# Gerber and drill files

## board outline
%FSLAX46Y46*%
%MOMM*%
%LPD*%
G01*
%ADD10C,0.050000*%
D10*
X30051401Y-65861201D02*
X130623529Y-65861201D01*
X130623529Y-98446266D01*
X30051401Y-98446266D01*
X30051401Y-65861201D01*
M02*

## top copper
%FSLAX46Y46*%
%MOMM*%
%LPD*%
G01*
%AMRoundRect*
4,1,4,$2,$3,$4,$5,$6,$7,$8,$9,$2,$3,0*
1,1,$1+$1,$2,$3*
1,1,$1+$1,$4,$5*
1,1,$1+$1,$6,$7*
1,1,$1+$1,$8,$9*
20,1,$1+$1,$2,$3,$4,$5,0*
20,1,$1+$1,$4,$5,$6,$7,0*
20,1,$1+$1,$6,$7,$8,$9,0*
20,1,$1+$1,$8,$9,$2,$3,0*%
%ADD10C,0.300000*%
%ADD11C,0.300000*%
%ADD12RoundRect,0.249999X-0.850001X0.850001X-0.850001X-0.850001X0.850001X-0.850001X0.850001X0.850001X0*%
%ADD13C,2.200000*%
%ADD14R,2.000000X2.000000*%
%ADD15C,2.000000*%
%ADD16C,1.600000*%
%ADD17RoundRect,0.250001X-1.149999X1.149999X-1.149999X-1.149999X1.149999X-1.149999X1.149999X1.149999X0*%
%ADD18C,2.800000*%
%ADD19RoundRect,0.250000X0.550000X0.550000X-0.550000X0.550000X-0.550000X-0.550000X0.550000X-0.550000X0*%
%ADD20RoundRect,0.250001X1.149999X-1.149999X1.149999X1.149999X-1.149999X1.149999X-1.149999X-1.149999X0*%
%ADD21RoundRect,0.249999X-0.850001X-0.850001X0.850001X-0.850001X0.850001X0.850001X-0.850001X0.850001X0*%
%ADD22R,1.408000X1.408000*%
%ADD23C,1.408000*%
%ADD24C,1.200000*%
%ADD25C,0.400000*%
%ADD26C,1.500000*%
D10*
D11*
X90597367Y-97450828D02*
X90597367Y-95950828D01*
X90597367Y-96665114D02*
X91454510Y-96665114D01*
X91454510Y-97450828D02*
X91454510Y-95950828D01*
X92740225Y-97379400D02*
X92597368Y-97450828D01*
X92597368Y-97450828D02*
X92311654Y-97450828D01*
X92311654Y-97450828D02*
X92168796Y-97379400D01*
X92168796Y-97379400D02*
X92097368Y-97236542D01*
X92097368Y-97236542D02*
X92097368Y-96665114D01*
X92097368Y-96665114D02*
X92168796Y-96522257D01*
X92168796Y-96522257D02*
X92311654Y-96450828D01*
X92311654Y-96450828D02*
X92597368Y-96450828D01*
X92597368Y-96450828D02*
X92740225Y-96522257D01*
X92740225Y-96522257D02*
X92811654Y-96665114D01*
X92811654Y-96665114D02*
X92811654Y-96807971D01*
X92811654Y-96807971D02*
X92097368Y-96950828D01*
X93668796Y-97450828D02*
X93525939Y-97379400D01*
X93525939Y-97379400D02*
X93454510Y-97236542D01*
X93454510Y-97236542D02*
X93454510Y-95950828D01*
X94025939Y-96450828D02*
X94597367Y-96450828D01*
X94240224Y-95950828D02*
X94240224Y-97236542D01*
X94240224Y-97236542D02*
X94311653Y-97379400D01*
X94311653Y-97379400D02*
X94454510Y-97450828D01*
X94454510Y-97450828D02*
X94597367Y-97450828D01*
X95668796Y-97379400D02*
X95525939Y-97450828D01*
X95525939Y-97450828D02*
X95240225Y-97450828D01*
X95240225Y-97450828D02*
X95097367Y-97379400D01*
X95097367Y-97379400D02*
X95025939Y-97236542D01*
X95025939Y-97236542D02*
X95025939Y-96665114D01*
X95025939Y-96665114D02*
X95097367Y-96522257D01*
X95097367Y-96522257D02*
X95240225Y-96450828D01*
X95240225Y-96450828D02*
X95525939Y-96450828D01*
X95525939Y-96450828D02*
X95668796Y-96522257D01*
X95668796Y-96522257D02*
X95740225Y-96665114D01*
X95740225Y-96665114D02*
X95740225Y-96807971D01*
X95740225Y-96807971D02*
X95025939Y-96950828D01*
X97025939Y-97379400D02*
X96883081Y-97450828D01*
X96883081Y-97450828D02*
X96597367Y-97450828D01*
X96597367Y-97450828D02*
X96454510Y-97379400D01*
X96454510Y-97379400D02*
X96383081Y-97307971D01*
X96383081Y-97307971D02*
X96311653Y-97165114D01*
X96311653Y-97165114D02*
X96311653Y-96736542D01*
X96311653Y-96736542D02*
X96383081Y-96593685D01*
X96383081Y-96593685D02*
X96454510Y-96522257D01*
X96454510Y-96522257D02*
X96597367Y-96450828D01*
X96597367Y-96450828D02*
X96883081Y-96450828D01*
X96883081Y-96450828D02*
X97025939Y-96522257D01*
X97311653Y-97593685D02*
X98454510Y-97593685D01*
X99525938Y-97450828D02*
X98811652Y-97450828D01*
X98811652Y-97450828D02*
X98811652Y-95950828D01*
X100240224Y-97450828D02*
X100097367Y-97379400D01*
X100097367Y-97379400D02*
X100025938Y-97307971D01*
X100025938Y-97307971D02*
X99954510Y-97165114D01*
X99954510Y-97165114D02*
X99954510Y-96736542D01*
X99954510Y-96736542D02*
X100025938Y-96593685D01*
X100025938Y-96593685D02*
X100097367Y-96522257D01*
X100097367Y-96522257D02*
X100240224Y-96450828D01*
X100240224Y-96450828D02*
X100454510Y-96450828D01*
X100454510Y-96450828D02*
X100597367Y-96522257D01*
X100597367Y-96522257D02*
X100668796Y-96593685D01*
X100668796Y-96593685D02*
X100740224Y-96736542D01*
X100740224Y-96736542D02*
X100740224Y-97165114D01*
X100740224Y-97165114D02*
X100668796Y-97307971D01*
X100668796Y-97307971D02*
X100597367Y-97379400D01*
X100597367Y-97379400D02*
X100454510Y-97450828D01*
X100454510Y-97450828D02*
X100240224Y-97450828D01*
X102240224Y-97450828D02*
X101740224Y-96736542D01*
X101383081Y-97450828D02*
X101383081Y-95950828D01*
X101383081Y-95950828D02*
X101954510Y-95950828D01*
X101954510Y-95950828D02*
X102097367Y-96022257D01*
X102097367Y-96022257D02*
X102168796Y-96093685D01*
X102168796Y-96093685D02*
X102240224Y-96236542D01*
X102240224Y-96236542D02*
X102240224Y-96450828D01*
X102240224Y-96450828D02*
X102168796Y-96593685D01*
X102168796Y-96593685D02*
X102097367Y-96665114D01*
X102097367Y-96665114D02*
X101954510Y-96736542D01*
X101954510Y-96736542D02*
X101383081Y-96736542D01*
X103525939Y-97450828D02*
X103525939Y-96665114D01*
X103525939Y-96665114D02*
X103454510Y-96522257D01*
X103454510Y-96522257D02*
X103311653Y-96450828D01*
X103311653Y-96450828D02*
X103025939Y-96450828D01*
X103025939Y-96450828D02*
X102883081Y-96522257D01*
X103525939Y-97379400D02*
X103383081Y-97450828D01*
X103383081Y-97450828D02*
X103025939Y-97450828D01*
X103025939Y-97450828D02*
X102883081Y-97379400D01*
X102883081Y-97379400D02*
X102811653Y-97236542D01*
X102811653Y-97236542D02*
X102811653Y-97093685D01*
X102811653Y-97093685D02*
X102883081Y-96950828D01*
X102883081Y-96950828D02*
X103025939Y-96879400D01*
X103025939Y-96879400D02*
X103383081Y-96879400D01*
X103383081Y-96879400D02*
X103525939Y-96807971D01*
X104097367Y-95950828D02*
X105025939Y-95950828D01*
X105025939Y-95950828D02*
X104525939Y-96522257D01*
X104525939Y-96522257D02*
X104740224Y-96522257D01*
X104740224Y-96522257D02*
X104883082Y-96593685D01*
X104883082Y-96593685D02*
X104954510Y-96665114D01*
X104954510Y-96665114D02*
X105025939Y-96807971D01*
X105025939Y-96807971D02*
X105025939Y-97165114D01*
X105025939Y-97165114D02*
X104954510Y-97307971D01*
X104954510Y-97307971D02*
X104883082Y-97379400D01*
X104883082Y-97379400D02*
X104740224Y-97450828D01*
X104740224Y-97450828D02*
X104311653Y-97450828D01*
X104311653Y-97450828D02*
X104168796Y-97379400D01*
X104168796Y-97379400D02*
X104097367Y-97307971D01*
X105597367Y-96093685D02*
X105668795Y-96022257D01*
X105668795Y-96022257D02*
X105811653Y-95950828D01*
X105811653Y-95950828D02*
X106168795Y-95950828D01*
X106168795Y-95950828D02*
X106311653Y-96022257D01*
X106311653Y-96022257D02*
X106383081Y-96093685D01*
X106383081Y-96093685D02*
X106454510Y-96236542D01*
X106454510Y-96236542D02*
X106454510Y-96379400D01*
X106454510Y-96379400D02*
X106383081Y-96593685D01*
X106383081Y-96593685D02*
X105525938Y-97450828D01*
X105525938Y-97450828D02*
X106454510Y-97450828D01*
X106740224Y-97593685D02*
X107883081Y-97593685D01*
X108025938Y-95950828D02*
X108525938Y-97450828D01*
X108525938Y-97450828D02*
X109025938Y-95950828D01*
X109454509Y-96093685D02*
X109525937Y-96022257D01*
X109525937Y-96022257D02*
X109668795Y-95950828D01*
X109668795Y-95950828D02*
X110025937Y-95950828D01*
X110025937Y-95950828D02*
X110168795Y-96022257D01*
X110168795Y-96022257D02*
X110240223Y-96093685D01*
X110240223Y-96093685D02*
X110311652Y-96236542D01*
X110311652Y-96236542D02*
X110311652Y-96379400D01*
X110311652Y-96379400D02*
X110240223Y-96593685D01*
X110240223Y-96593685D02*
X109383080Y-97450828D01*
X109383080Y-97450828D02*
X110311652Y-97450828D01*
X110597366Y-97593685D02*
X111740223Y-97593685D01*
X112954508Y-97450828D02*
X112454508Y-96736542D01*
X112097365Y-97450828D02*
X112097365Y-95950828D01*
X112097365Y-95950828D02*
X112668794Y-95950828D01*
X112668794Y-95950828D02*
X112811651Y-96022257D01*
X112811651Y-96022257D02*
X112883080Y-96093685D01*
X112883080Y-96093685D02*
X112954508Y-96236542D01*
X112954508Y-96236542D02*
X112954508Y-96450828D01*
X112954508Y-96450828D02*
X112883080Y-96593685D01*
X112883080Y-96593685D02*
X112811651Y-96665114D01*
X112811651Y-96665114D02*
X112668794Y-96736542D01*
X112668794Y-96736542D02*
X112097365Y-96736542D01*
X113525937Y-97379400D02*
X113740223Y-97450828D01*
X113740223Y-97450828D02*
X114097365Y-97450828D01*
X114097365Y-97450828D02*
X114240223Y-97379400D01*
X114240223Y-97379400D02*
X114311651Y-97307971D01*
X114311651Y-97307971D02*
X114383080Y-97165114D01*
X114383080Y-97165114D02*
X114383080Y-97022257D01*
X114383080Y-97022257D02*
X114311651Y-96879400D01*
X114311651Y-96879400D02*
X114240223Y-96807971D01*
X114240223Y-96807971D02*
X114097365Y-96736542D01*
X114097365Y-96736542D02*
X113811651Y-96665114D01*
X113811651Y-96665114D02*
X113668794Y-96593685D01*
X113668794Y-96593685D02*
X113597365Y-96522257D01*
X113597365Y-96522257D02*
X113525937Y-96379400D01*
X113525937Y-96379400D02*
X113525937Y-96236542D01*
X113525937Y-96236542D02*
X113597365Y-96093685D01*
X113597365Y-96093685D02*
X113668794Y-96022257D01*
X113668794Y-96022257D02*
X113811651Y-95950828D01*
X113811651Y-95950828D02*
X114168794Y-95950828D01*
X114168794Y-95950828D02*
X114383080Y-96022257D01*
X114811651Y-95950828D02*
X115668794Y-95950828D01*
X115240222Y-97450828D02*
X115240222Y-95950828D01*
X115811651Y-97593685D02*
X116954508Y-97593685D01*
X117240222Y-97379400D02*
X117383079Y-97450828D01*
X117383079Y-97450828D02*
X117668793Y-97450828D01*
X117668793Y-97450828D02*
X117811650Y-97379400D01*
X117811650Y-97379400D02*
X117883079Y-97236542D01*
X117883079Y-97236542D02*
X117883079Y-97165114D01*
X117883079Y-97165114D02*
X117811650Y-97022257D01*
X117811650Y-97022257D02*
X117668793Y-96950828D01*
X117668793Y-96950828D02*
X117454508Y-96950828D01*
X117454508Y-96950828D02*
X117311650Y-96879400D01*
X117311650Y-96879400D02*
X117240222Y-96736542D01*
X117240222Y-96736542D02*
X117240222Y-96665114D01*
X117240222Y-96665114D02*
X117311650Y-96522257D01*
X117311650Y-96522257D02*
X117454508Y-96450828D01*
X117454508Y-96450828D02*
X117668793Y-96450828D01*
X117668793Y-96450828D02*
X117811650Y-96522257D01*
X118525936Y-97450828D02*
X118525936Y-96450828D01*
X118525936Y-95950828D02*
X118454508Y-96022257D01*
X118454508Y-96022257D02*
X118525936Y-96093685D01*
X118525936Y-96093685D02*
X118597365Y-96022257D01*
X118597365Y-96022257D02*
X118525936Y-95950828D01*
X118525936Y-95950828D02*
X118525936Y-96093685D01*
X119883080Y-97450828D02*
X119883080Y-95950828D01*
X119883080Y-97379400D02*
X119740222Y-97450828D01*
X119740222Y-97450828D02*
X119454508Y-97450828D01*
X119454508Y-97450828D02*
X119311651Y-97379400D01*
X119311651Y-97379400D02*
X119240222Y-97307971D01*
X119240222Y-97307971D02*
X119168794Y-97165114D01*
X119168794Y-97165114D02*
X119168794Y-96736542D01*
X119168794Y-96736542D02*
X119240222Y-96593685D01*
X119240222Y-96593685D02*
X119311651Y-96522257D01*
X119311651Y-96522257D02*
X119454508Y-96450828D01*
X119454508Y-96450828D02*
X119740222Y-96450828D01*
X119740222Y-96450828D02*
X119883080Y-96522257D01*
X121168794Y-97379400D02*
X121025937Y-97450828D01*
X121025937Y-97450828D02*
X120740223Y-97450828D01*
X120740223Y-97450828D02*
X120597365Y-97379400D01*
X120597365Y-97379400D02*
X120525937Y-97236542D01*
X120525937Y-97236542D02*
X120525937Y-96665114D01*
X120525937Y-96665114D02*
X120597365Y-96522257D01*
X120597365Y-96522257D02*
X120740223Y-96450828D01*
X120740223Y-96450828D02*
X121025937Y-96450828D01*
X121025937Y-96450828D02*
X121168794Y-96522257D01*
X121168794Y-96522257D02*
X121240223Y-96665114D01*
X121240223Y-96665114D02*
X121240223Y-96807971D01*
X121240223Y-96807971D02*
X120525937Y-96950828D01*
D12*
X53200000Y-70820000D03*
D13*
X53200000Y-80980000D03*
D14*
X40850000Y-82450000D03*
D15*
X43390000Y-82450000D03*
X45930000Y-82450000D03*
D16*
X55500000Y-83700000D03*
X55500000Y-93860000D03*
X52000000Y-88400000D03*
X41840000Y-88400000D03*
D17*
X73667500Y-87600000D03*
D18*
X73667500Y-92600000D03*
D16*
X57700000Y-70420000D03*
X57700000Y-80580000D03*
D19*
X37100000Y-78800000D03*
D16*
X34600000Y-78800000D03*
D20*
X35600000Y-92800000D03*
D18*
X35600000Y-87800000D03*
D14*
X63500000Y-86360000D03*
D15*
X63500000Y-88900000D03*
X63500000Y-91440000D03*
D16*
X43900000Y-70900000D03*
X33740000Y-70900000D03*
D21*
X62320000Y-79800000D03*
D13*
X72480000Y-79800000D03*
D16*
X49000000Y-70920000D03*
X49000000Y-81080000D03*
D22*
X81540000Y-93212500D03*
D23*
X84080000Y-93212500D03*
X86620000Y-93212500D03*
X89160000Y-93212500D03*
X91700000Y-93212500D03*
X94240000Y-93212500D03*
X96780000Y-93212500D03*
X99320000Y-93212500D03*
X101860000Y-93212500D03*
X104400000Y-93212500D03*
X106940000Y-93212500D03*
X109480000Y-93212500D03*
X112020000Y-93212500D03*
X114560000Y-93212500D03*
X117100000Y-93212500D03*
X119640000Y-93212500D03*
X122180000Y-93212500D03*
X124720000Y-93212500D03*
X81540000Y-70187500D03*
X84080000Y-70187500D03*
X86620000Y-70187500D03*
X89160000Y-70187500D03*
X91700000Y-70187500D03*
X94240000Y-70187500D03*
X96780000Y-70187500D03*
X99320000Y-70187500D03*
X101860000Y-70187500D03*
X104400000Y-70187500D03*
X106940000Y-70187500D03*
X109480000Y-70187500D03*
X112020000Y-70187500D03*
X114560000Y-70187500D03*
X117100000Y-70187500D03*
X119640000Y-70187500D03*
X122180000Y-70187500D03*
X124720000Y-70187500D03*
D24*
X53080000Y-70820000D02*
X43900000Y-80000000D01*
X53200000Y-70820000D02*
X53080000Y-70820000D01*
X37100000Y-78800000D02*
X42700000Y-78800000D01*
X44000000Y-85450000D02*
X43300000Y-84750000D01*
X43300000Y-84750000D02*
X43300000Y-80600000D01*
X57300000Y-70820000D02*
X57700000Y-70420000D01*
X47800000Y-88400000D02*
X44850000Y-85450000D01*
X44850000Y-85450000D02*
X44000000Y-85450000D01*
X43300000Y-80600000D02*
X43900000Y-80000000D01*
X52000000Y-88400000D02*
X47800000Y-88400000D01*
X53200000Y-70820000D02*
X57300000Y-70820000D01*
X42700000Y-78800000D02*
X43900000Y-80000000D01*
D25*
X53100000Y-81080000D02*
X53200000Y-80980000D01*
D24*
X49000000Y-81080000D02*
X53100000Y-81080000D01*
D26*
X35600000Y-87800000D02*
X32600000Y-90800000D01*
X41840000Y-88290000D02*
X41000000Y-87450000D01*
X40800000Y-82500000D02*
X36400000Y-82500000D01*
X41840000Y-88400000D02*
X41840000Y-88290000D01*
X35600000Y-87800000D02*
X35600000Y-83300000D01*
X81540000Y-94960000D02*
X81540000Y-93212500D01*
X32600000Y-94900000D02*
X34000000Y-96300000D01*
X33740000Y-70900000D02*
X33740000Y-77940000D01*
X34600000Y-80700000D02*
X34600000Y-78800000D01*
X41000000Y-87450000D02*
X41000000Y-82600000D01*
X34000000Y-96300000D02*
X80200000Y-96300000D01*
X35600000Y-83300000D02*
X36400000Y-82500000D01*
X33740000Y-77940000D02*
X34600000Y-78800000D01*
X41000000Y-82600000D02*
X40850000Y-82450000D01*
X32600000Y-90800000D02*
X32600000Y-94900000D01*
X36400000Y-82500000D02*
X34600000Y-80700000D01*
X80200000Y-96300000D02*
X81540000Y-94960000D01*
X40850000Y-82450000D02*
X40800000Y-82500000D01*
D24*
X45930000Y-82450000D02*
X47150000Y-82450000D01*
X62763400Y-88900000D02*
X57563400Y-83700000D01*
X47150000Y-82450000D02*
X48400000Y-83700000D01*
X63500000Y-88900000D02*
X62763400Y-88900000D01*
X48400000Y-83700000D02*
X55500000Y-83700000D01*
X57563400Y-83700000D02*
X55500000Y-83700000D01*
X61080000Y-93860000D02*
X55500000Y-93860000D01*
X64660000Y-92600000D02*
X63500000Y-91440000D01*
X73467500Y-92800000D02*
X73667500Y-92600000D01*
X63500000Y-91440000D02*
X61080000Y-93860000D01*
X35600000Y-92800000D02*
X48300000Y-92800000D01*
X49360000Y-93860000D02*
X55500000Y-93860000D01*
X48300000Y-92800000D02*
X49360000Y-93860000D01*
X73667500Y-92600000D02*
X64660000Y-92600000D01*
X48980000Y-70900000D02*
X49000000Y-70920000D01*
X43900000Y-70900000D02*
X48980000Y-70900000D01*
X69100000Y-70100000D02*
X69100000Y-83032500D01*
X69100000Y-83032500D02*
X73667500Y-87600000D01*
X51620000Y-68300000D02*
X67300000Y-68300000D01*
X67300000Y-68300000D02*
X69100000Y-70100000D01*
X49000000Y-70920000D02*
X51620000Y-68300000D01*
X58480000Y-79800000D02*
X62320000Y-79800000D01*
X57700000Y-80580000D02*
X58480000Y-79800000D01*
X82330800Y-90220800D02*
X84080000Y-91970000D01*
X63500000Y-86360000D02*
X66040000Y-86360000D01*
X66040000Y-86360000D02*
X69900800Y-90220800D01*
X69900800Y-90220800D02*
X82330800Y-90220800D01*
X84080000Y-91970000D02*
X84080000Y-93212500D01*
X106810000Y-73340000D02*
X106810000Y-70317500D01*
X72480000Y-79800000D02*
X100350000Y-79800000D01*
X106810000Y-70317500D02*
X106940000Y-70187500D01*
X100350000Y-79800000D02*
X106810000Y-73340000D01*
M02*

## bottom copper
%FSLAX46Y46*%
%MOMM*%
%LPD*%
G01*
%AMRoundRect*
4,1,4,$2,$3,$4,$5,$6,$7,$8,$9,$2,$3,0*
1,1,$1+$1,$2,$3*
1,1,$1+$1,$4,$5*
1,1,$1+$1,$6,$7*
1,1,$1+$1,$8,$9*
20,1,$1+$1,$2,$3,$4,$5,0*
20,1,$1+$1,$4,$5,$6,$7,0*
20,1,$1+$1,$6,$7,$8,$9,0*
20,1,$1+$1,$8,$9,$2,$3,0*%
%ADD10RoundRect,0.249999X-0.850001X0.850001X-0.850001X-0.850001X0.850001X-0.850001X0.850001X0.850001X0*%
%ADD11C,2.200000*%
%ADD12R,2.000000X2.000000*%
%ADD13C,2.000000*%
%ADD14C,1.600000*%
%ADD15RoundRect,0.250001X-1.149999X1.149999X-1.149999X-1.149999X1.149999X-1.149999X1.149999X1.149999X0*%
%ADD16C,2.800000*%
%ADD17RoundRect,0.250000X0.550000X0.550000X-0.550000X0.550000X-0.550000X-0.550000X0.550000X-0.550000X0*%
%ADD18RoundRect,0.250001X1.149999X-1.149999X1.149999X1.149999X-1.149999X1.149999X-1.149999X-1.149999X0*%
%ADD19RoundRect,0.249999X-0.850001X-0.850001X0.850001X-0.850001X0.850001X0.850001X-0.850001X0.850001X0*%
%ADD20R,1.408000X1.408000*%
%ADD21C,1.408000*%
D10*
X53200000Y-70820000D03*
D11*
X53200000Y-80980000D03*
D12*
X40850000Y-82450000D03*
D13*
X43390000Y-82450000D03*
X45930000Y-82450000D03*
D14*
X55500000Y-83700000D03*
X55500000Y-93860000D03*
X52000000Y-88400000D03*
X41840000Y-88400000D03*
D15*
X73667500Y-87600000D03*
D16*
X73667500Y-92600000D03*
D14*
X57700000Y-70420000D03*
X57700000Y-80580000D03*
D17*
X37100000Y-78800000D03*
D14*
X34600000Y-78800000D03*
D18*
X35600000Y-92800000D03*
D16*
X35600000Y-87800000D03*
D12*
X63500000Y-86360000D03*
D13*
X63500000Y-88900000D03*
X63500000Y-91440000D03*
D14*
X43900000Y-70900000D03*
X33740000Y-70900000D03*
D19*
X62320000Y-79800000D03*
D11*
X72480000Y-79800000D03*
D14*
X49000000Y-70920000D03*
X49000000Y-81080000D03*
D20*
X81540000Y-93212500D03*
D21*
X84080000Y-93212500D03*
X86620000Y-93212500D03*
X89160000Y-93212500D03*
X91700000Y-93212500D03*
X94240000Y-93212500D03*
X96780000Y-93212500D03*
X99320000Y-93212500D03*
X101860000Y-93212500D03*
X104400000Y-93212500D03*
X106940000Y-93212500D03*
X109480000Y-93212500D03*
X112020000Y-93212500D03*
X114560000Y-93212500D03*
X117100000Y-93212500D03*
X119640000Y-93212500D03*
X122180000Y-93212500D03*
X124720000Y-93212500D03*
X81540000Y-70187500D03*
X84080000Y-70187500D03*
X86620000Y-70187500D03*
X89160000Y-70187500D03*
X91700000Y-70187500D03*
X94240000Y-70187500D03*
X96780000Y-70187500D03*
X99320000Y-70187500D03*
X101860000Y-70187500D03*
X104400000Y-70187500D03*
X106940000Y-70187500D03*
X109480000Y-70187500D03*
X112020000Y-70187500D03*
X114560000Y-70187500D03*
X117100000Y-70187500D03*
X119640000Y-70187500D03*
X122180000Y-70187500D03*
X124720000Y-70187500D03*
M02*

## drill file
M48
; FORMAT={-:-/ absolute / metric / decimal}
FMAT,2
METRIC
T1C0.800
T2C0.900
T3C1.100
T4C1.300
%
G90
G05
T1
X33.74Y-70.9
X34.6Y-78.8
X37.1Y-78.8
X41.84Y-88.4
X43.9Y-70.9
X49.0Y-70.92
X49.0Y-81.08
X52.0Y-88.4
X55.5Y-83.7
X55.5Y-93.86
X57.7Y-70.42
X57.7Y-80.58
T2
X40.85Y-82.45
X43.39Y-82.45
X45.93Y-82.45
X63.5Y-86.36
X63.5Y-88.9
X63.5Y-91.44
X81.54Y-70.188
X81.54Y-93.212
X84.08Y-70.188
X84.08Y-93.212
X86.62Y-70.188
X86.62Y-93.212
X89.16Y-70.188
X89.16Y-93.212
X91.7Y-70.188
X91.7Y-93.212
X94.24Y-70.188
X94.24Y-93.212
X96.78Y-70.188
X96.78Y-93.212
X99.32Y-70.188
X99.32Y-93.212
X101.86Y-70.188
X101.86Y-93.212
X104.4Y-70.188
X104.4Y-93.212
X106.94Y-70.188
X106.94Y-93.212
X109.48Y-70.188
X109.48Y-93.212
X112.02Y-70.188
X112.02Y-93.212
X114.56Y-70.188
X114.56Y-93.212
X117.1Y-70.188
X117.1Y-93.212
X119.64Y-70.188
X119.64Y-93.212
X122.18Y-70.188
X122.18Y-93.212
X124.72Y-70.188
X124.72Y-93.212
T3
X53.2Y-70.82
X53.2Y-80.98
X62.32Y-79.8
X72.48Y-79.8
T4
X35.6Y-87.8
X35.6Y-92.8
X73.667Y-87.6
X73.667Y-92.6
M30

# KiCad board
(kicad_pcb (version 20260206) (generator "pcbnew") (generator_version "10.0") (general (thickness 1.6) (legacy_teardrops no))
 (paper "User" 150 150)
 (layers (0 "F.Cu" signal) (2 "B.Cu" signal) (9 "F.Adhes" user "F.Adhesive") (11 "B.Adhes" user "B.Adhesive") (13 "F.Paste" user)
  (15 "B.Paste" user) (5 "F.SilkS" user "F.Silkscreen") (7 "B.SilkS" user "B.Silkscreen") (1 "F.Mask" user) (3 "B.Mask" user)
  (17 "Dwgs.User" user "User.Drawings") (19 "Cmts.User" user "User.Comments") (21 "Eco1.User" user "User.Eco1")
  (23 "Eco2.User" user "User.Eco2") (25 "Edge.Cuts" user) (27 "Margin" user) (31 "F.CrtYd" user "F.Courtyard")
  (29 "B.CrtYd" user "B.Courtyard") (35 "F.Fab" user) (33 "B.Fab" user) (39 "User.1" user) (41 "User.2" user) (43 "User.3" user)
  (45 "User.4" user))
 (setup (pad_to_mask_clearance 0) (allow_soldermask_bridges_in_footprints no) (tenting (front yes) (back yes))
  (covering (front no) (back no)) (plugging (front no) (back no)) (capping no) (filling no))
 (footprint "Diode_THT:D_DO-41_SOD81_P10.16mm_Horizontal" (layer "F.Cu") (at 53.2 70.82 -90)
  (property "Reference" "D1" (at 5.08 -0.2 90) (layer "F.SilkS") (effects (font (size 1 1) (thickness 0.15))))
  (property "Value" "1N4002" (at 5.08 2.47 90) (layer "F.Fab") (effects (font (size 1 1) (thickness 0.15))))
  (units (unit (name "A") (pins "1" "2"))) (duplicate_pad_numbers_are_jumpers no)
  (pad "1" thru_hole roundrect (at 0 0 270) (size 2.2 2.2) (drill 1.1) (layers "*.Cu" "*.Mask") (remove_unused_layers no)
   (roundrect_rratio 0.113636) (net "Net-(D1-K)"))
  (pad "2" thru_hole circle (at 10.16 0 270) (size 2.2 2.2) (drill 1.1) (layers "*.Cu" "*.Mask") (remove_unused_layers no)
   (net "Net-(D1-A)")))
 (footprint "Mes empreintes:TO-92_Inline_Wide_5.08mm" (layer "F.Cu") (at 40.85 82.45)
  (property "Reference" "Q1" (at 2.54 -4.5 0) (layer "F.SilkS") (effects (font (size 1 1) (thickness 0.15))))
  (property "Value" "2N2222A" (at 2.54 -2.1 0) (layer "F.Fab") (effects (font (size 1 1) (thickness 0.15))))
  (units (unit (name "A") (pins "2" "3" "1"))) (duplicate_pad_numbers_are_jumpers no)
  (pad "1" thru_hole rect (at 0 0) (size 2 2) (drill 0.9) (layers "*.Cu" "*.Mask") (remove_unused_layers no) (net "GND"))
  (pad "2" thru_hole circle (at 2.54 0) (size 2 2) (drill 0.9) (layers "*.Cu" "*.Mask") (remove_unused_layers no) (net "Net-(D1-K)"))
  (pad "3" thru_hole circle (at 5.08 0) (size 2 2) (drill 0.9) (layers "*.Cu" "*.Mask") (remove_unused_layers no) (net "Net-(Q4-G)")))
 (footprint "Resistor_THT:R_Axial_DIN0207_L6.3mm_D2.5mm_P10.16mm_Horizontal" (layer "F.Cu") (at 55.5 83.7 -90)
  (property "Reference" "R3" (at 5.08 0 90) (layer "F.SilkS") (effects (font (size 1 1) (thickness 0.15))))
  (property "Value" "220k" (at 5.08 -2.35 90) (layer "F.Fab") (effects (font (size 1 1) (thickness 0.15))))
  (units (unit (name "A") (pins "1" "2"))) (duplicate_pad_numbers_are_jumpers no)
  (pad "1" thru_hole circle (at 0 0 270) (size 1.6 1.6) (drill 0.8) (layers "*.Cu" "*.Mask") (remove_unused_layers no) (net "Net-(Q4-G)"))
  (pad "2" thru_hole circle (at 10.16 0 270) (size 1.6 1.6) (drill 0.8) (layers "*.Cu" "*.Mask") (remove_unused_layers no) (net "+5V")))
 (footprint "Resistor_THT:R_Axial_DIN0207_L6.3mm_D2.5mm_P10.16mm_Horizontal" (layer "F.Cu") (at 52 88.4 180)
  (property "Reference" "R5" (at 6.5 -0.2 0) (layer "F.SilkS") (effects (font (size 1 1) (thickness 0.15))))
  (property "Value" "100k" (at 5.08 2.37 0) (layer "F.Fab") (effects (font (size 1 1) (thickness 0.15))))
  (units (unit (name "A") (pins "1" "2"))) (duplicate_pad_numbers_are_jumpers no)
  (pad "1" thru_hole circle (at 0 0 180) (size 1.6 1.6) (drill 0.8) (layers "*.Cu" "*.Mask") (remove_unused_layers no) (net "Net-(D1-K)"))
  (pad "2" thru_hole circle (at 10.16 0 180) (size 1.6 1.6) (drill 0.8) (layers "*.Cu" "*.Mask") (remove_unused_layers no) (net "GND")))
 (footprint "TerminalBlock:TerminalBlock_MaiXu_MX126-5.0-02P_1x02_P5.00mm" (layer "F.Cu") (at 73.6675 87.6 -90)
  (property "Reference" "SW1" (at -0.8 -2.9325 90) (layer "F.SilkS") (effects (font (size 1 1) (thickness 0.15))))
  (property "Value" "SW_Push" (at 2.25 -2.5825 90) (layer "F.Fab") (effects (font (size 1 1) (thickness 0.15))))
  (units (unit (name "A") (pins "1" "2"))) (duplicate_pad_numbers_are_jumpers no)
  (pad "1" thru_hole roundrect (at 0 0 270) (size 2.8 2.8) (drill 1.3) (layers "*.Cu" "*.Mask") (remove_unused_layers no)
   (roundrect_rratio 0.089286) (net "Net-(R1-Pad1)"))
  (pad "2" thru_hole circle (at 5 0 270) (size 2.8 2.8) (drill 1.3) (layers "*.Cu" "*.Mask") (remove_unused_layers no) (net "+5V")))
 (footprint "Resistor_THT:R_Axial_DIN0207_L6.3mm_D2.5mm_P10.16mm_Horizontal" (layer "F.Cu") (at 57.7 70.42 -90)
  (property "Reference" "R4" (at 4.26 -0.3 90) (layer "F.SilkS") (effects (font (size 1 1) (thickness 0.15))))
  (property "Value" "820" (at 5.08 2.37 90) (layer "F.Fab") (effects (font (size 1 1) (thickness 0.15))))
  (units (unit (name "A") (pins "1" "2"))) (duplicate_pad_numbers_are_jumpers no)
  (pad "1" thru_hole circle (at 0 0 270) (size 1.6 1.6) (drill 0.8) (layers "*.Cu" "*.Mask") (remove_unused_layers no) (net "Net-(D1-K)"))
  (pad "2" thru_hole circle (at 10.16 0 270) (size 1.6 1.6) (drill 0.8) (layers "*.Cu" "*.Mask") (remove_unused_layers no)
   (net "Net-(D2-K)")))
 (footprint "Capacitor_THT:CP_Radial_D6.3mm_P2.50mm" (layer "F.Cu") (at 37.1 78.8 180)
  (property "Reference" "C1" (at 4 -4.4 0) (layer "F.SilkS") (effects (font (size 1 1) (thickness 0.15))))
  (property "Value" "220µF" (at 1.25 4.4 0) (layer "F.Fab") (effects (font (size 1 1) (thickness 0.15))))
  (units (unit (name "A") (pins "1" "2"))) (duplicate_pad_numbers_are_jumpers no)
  (pad "1" thru_hole roundrect (at 0 0 180) (size 1.6 1.6) (drill 0.8) (layers "*.Cu" "*.Mask") (remove_unused_layers no)
   (roundrect_rratio 0.15625) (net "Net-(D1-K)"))
  (pad "2" thru_hole circle (at 2.5 0 180) (size 1.6 1.6) (drill 0.8) (layers "*.Cu" "*.Mask") (remove_unused_layers no) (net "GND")))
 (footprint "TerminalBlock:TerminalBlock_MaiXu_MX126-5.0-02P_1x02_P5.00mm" (layer "F.Cu") (at 35.6 92.8 90)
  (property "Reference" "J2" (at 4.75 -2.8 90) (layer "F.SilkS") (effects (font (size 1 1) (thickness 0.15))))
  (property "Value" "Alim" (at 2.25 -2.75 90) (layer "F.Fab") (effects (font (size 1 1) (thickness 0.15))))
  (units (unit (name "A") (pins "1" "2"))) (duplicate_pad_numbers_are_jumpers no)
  (pad "1" thru_hole roundrect (at 0 0 90) (size 2.8 2.8) (drill 1.3) (layers "*.Cu" "*.Mask") (remove_unused_layers no)
   (roundrect_rratio 0.089286) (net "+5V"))
  (pad "2" thru_hole circle (at 5 0 90) (size 2.8 2.8) (drill 1.3) (layers "*.Cu" "*.Mask") (remove_unused_layers no) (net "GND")))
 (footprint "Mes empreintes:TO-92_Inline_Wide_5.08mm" (layer "F.Cu") (at 63.5 86.36 -90)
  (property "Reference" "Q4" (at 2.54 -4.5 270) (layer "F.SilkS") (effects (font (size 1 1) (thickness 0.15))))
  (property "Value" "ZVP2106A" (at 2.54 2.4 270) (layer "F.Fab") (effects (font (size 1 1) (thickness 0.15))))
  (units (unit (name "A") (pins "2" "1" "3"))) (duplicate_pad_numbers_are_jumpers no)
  (pad "1" thru_hole rect (at 0 0 270) (size 2 2) (drill 0.9) (layers "*.Cu" "*.Mask") (remove_unused_layers no) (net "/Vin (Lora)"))
  (pad "2" thru_hole circle (at 2.54 0 270) (size 2 2) (drill 0.9) (layers "*.Cu" "*.Mask") (remove_unused_layers no) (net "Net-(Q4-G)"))
  (pad "3" thru_hole circle (at 5.08 0 270) (size 2 2) (drill 0.9) (layers "*.Cu" "*.Mask") (remove_unused_layers no) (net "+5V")))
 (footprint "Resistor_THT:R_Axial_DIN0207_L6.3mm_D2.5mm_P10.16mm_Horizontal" (layer "F.Cu") (at 43.9 70.9 180)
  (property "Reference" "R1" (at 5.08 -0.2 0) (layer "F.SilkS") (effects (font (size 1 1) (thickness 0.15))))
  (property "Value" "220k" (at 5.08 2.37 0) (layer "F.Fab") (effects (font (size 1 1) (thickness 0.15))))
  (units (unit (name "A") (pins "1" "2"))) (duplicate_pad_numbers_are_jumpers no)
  (pad "1" thru_hole circle (at 0 0 180) (size 1.6 1.6) (drill 0.8) (layers "*.Cu" "*.Mask") (remove_unused_layers no) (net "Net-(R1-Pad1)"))
  (pad "2" thru_hole circle (at 10.16 0 180) (size 1.6 1.6) (drill 0.8) (layers "*.Cu" "*.Mask") (remove_unused_layers no) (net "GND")))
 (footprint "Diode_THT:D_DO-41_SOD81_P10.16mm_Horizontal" (layer "F.Cu") (at 62.32 79.8)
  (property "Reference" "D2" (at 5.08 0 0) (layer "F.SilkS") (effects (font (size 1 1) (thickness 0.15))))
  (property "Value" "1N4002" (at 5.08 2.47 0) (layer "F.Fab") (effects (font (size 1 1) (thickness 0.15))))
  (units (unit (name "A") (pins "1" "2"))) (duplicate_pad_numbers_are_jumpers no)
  (pad "1" thru_hole roundrect (at 0 0) (size 2.2 2.2) (drill 1.1) (layers "*.Cu" "*.Mask") (remove_unused_layers no)
   (roundrect_rratio 0.113636) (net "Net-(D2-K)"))
  (pad "2" thru_hole circle (at 10.16 0) (size 2.2 2.2) (drill 1.1) (layers "*.Cu" "*.Mask") (remove_unused_layers no)
   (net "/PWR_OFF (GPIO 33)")))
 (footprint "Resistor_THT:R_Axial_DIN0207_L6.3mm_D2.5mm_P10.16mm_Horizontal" (layer "F.Cu") (at 49 70.92 -90)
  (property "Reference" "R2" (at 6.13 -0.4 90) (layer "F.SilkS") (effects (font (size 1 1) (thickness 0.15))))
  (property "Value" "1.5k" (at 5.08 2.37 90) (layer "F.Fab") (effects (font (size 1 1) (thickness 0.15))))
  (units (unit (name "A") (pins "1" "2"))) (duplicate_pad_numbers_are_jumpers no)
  (pad "1" thru_hole circle (at 0 0 270) (size 1.6 1.6) (drill 0.8) (layers "*.Cu" "*.Mask") (remove_unused_layers no) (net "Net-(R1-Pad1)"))
  (pad "2" thru_hole circle (at 10.16 0 270) (size 1.6 1.6) (drill 0.8) (layers "*.Cu" "*.Mask") (remove_unused_layers no)
   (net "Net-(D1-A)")))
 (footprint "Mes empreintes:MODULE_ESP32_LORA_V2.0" (layer "F.Cu") (at 103.92 81.7)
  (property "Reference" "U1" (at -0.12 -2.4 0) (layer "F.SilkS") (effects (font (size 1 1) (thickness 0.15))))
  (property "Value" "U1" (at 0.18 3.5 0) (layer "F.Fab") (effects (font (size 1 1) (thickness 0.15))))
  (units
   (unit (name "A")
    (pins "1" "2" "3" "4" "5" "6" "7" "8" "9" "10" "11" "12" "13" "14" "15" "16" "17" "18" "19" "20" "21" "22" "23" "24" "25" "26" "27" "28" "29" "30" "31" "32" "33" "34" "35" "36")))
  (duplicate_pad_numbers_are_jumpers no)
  (pad "1" thru_hole rect (at -22.38 11.5125) (size 1.408 1.408) (drill 0.9) (layers "*.Cu" "*.Mask") (remove_unused_layers no) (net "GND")
   (solder_mask_margin 0.102))
  (pad "2" thru_hole circle (at -19.84 11.5125) (size 1.408 1.408) (drill 0.9) (layers "*.Cu" "*.Mask") (remove_unused_layers no)
   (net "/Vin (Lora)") (solder_mask_margin 0.102))
  (pad "3" thru_hole circle (at -17.3 11.5125) (size 1.408 1.408) (drill 0.9) (layers "*.Cu" "*.Mask") (remove_unused_layers no)
   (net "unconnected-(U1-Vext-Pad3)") (solder_mask_margin 0.102))
  (pad "4" thru_hole circle (at -14.76 11.5125) (size 1.408 1.408) (drill 0.9) (layers "*.Cu" "*.Mask") (remove_unused_layers no)
   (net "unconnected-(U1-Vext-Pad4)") (solder_mask_margin 0.102))
  (pad "5" thru_hole circle (at -12.22 11.5125) (size 1.408 1.408) (drill 0.9) (layers "*.Cu" "*.Mask") (remove_unused_layers no)
   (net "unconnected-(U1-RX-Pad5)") (solder_mask_margin 0.102))
  (pad "6" thru_hole circle (at -9.68 11.5125) (size 1.408 1.408) (drill 0.9) (layers "*.Cu" "*.Mask") (remove_unused_layers no)
   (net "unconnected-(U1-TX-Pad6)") (solder_mask_margin 0.102))
  (pad "7" thru_hole circle (at -7.14 11.5125) (size 1.408 1.408) (drill 0.9) (layers "*.Cu" "*.Mask") (remove_unused_layers no)
   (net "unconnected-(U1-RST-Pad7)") (solder_mask_margin 0.102))
  (pad "8" thru_hole circle (at -4.6 11.5125) (size 1.408 1.408) (drill 0.9) (layers "*.Cu" "*.Mask") (remove_unused_layers no)
   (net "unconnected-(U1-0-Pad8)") (solder_mask_margin 0.102))
  (pad "9" thru_hole circle (at -2.06 11.5125) (size 1.408 1.408) (drill 0.9) (layers "*.Cu" "*.Mask") (remove_unused_layers no)
   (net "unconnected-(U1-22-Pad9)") (solder_mask_margin 0.102))
  (pad "10" thru_hole circle (at 0.48 11.5125) (size 1.408 1.408) (drill 0.9) (layers "*.Cu" "*.Mask") (remove_unused_layers no)
   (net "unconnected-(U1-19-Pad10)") (solder_mask_margin 0.102))
  (pad "11" thru_hole circle (at 3.02 11.5125) (size 1.408 1.408) (drill 0.9) (layers "*.Cu" "*.Mask") (remove_unused_layers no)
   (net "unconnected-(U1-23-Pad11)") (solder_mask_margin 0.102))
  (pad "12" thru_hole circle (at 5.56 11.5125) (size 1.408 1.408) (drill 0.9) (layers "*.Cu" "*.Mask") (remove_unused_layers no)
   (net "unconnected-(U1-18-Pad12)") (solder_mask_margin 0.102))
  (pad "13" thru_hole circle (at 8.1 11.5125) (size 1.408 1.408) (drill 0.9) (layers "*.Cu" "*.Mask") (remove_unused_layers no)
   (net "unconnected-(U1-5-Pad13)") (solder_mask_margin 0.102))
  (pad "14" thru_hole circle (at 10.64 11.5125) (size 1.408 1.408) (drill 0.9) (layers "*.Cu" "*.Mask") (remove_unused_layers no)
   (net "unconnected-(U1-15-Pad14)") (solder_mask_margin 0.102))
  (pad "15" thru_hole circle (at 13.18 11.5125) (size 1.408 1.408) (drill 0.9) (layers "*.Cu" "*.Mask") (remove_unused_layers no)
   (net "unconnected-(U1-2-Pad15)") (solder_mask_margin 0.102))
  (pad "16" thru_hole circle (at 15.72 11.5125) (size 1.408 1.408) (drill 0.9) (layers "*.Cu" "*.Mask") (remove_unused_layers no)
   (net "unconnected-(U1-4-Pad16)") (solder_mask_margin 0.102))
  (pad "17" thru_hole circle (at 18.26 11.5125) (size 1.408 1.408) (drill 0.9) (layers "*.Cu" "*.Mask") (remove_unused_layers no)
   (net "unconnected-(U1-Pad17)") (solder_mask_margin 0.102))
  (pad "18" thru_hole circle (at 20.8 11.5125) (size 1.408 1.408) (drill 0.9) (layers "*.Cu" "*.Mask") (remove_unused_layers no)
   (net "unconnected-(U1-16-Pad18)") (solder_mask_margin 0.102))
  (pad "19" thru_hole circle (at -22.38 -11.5125) (size 1.408 1.408) (drill 0.9) (layers "*.Cu" "*.Mask") (remove_unused_layers no)
   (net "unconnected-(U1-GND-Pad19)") (solder_mask_margin 0.102))
  (pad "20" thru_hole circle (at -19.84 -11.5125) (size 1.408 1.408) (drill 0.9) (layers "*.Cu" "*.Mask") (remove_unused_layers no)
   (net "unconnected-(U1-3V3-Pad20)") (solder_mask_margin 0.102))
  (pad "21" thru_hole circle (at -17.3 -11.5125) (size 1.408 1.408) (drill 0.9) (layers "*.Cu" "*.Mask") (remove_unused_layers no)
   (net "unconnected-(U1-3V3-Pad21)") (solder_mask_margin 0.102))
  (pad "22" thru_hole circle (at -14.76 -11.5125) (size 1.408 1.408) (drill 0.9) (layers "*.Cu" "*.Mask") (remove_unused_layers no)
   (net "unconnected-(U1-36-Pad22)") (solder_mask_margin 0.102))
  (pad "23" thru_hole circle (at -12.22 -11.5125) (size 1.408 1.408) (drill 0.9) (layers "*.Cu" "*.Mask") (remove_unused_layers no)
   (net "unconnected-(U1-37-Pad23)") (solder_mask_margin 0.102))
  (pad "24" thru_hole circle (at -9.68 -11.5125) (size 1.408 1.408) (drill 0.9) (layers "*.Cu" "*.Mask") (remove_unused_layers no)
   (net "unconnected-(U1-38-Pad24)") (solder_mask_margin 0.102))
  (pad "25" thru_hole circle (at -7.14 -11.5125) (size 1.408 1.408) (drill 0.9) (layers "*.Cu" "*.Mask") (remove_unused_layers no)
   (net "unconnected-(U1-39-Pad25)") (solder_mask_margin 0.102))
  (pad "26" thru_hole circle (at -4.6 -11.5125) (size 1.408 1.408) (drill 0.9) (layers "*.Cu" "*.Mask") (remove_unused_layers no)
   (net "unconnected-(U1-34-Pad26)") (solder_mask_margin 0.102))
  (pad "27" thru_hole circle (at -2.06 -11.5125) (size 1.408 1.408) (drill 0.9) (layers "*.Cu" "*.Mask") (remove_unused_layers no)
   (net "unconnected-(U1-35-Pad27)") (solder_mask_margin 0.102))
  (pad "28" thru_hole circle (at 0.48 -11.5125) (size 1.408 1.408) (drill 0.9) (layers "*.Cu" "*.Mask") (remove_unused_layers no)
   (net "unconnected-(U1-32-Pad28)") (solder_mask_margin 0.102))
  (pad "29" thru_hole circle (at 3.02 -11.5125) (size 1.408 1.408) (drill 0.9) (layers "*.Cu" "*.Mask") (remove_unused_layers no)
   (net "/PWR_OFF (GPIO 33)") (solder_mask_margin 0.102))
  (pad "30" thru_hole circle (at 5.56 -11.5125) (size 1.408 1.408) (drill 0.9) (layers "*.Cu" "*.Mask") (remove_unused_layers no)
   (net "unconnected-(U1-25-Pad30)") (solder_mask_margin 0.102))
  (pad "31" thru_hole circle (at 8.1 -11.5125) (size 1.408 1.408) (drill 0.9) (layers "*.Cu" "*.Mask") (remove_unused_layers no)
   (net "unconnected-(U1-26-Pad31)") (solder_mask_margin 0.102))
  (pad "32" thru_hole circle (at 10.64 -11.5125) (size 1.408 1.408) (drill 0.9) (layers "*.Cu" "*.Mask") (remove_unused_layers no)
   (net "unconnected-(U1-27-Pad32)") (solder_mask_margin 0.102))
  (pad "33" thru_hole circle (at 13.18 -11.5125) (size 1.408 1.408) (drill 0.9) (layers "*.Cu" "*.Mask") (remove_unused_layers no)
   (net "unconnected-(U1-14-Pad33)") (solder_mask_margin 0.102))
  (pad "34" thru_hole circle (at 15.72 -11.5125) (size 1.408 1.408) (drill 0.9) (layers "*.Cu" "*.Mask") (remove_unused_layers no)
   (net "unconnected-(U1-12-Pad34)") (solder_mask_margin 0.102))
  (pad "35" thru_hole circle (at 18.26 -11.5125) (size 1.408 1.408) (drill 0.9) (layers "*.Cu" "*.Mask") (remove_unused_layers no)
   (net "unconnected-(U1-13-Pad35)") (solder_mask_margin 0.102))
  (pad "36" thru_hole circle (at 20.8 -11.5125) (size 1.408 1.408) (drill 0.9) (layers "*.Cu" "*.Mask") (remove_unused_layers no)
   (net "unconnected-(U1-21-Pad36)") (solder_mask_margin 0.102)))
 (gr_rect (start 30.051401 65.861201) (end 130.623529 98.446266) (stroke (width 0.05) (type default)) (fill no) (layer "Edge.Cuts"))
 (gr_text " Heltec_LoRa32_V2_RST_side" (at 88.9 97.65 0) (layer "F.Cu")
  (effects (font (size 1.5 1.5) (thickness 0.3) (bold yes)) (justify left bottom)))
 (segment (start 53.08 70.82) (end 43.9 80) (width 1.2) (layer "F.Cu") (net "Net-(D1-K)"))
 (segment (start 53.2 70.82) (end 53.08 70.82) (width 1.2) (layer "F.Cu") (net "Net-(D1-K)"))
 (segment (start 37.1 78.8) (end 42.7 78.8) (width 1.2) (layer "F.Cu") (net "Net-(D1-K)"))
 (segment (start 44 85.45) (end 43.3 84.75) (width 1.2) (layer "F.Cu") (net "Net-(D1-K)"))
 (segment (start 43.3 84.75) (end 43.3 80.6) (width 1.2) (layer "F.Cu") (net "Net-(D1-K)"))
 (segment (start 57.3 70.82) (end 57.7 70.42) (width 1.2) (layer "F.Cu") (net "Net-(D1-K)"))
 (segment (start 47.8 88.4) (end 44.85 85.45) (width 1.2) (layer "F.Cu") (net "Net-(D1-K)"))
 (segment (start 44.85 85.45) (end 44 85.45) (width 1.2) (layer "F.Cu") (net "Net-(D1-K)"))
 (segment (start 43.3 80.6) (end 43.9 80) (width 1.2) (layer "F.Cu") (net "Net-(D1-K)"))
 (segment (start 52 88.4) (end 47.8 88.4) (width 1.2) (layer "F.Cu") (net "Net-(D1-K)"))
 (segment (start 53.2 70.82) (end 57.3 70.82) (width 1.2) (layer "F.Cu") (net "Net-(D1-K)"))
 (segment (start 42.7 78.8) (end 43.9 80) (width 1.2) (layer "F.Cu") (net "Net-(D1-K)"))
 (segment (start 53.1 81.08) (end 53.2 80.98) (width 0.4) (layer "F.Cu") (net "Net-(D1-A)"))
 (segment (start 49 81.08) (end 53.1 81.08) (width 1.2) (layer "F.Cu") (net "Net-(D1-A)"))
 (segment (start 35.6 87.8) (end 32.6 90.8) (width 1.5) (layer "F.Cu") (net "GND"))
 (segment (start 41.84 88.29) (end 41 87.45) (width 1.5) (layer "F.Cu") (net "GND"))
 (segment (start 40.8 82.5) (end 36.4 82.5) (width 1.5) (layer "F.Cu") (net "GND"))
 (segment (start 41.84 88.4) (end 41.84 88.29) (width 1.5) (layer "F.Cu") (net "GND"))
 (segment (start 35.6 87.8) (end 35.6 83.3) (width 1.5) (layer "F.Cu") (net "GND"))
 (segment (start 81.54 94.96) (end 81.54 93.2125) (width 1.5) (layer "F.Cu") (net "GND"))
 (segment (start 32.6 94.9) (end 34 96.3) (width 1.5) (layer "F.Cu") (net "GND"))
 (segment (start 33.74 70.9) (end 33.74 77.94) (width 1.5) (layer "F.Cu") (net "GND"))
 (segment (start 34.6 80.7) (end 34.6 78.8) (width 1.5) (layer "F.Cu") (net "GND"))
 (segment (start 41 87.45) (end 41 82.6) (width 1.5) (layer "F.Cu") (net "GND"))
 (segment (start 34 96.3) (end 80.2 96.3) (width 1.5) (layer "F.Cu") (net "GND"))
 (segment (start 35.6 83.3) (end 36.4 82.5) (width 1.5) (layer "F.Cu") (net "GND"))
 (segment (start 33.74 77.94) (end 34.6 78.8) (width 1.5) (layer "F.Cu") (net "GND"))
 (segment (start 41 82.6) (end 40.85 82.45) (width 1.5) (layer "F.Cu") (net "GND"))
 (segment (start 32.6 90.8) (end 32.6 94.9) (width 1.5) (layer "F.Cu") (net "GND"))
 (segment (start 36.4 82.5) (end 34.6 80.7) (width 1.5) (layer "F.Cu") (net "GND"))
 (segment (start 80.2 96.3) (end 81.54 94.96) (width 1.5) (layer "F.Cu") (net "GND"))
 (segment (start 40.85 82.45) (end 40.8 82.5) (width 1.5) (layer "F.Cu") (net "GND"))
 (segment (start 45.93 82.45) (end 47.15 82.45) (width 1.2) (layer "F.Cu") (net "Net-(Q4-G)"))
 (segment (start 62.7634 88.9) (end 57.5634 83.7) (width 1.2) (layer "F.Cu") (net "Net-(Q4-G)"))
 (segment (start 47.15 82.45) (end 48.4 83.7) (width 1.2) (layer "F.Cu") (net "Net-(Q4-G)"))
 (segment (start 63.5 88.9) (end 62.7634 88.9) (width 1.2) (layer "F.Cu") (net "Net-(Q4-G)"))
 (segment (start 48.4 83.7) (end 55.5 83.7) (width 1.2) (layer "F.Cu") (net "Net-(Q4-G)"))
 (segment (start 57.5634 83.7) (end 55.5 83.7) (width 1.2) (layer "F.Cu") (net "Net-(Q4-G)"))
 (segment (start 61.08 93.86) (end 55.5 93.86) (width 1.2) (layer "F.Cu") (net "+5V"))
 (segment (start 64.66 92.6) (end 63.5 91.44) (width 1.2) (layer "F.Cu") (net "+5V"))
 (segment (start 73.4675 92.8) (end 73.6675 92.6) (width 1.2) (layer "F.Cu") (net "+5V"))
 (segment (start 63.5 91.44) (end 61.08 93.86) (width 1.2) (layer "F.Cu") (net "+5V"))
 (segment (start 35.6 92.8) (end 48.3 92.8) (width 1.2) (layer "F.Cu") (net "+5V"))
 (segment (start 49.36 93.86) (end 55.5 93.86) (width 1.2) (layer "F.Cu") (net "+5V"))
 (segment (start 48.3 92.8) (end 49.36 93.86) (width 1.2) (layer "F.Cu") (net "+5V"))
 (segment (start 73.6675 92.6) (end 64.66 92.6) (width 1.2) (layer "F.Cu") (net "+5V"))
 (segment (start 48.98 70.9) (end 49 70.92) (width 1.2) (layer "F.Cu") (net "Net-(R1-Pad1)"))
 (segment (start 43.9 70.9) (end 48.98 70.9) (width 1.2) (layer "F.Cu") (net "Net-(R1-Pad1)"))
 (segment (start 69.1 70.1) (end 69.1 83.0325) (width 1.2) (layer "F.Cu") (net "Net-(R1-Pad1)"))
 (segment (start 69.1 83.0325) (end 73.6675 87.6) (width 1.2) (layer "F.Cu") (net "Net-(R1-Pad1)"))
 (segment (start 51.62 68.3) (end 67.3 68.3) (width 1.2) (layer "F.Cu") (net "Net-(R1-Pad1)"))
 (segment (start 67.3 68.3) (end 69.1 70.1) (width 1.2) (layer "F.Cu") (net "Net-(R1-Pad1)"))
 (segment (start 49 70.92) (end 51.62 68.3) (width 1.2) (layer "F.Cu") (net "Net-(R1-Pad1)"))
 (segment (start 58.48 79.8) (end 62.32 79.8) (width 1.2) (layer "F.Cu") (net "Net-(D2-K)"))
 (segment (start 57.7 80.58) (end 58.48 79.8) (width 1.2) (layer "F.Cu") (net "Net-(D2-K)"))
 (segment (start 82.3308 90.2208) (end 84.08 91.97) (width 1.2) (layer "F.Cu") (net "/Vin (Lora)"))
 (segment (start 63.5 86.36) (end 66.04 86.36) (width 1.2) (layer "F.Cu") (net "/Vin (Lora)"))
 (segment (start 66.04 86.36) (end 69.9008 90.2208) (width 1.2) (layer "F.Cu") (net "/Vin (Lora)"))
 (segment (start 69.9008 90.2208) (end 82.3308 90.2208) (width 1.2) (layer "F.Cu") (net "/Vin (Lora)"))
 (segment (start 84.08 91.97) (end 84.08 93.2125) (width 1.2) (layer "F.Cu") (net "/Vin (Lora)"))
 (segment (start 106.81 73.34) (end 106.81 70.3175) (width 1.2) (layer "F.Cu") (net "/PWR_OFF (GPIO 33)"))
 (segment (start 72.48 79.8) (end 100.35 79.8) (width 1.2) (layer "F.Cu") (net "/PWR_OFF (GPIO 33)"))
 (segment (start 106.81 70.3175) (end 106.94 70.1875) (width 1.2) (layer "F.Cu") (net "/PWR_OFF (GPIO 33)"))
 (segment (start 100.35 79.8) (end 106.81 73.34) (width 1.2) (layer "F.Cu") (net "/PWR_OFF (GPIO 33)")))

